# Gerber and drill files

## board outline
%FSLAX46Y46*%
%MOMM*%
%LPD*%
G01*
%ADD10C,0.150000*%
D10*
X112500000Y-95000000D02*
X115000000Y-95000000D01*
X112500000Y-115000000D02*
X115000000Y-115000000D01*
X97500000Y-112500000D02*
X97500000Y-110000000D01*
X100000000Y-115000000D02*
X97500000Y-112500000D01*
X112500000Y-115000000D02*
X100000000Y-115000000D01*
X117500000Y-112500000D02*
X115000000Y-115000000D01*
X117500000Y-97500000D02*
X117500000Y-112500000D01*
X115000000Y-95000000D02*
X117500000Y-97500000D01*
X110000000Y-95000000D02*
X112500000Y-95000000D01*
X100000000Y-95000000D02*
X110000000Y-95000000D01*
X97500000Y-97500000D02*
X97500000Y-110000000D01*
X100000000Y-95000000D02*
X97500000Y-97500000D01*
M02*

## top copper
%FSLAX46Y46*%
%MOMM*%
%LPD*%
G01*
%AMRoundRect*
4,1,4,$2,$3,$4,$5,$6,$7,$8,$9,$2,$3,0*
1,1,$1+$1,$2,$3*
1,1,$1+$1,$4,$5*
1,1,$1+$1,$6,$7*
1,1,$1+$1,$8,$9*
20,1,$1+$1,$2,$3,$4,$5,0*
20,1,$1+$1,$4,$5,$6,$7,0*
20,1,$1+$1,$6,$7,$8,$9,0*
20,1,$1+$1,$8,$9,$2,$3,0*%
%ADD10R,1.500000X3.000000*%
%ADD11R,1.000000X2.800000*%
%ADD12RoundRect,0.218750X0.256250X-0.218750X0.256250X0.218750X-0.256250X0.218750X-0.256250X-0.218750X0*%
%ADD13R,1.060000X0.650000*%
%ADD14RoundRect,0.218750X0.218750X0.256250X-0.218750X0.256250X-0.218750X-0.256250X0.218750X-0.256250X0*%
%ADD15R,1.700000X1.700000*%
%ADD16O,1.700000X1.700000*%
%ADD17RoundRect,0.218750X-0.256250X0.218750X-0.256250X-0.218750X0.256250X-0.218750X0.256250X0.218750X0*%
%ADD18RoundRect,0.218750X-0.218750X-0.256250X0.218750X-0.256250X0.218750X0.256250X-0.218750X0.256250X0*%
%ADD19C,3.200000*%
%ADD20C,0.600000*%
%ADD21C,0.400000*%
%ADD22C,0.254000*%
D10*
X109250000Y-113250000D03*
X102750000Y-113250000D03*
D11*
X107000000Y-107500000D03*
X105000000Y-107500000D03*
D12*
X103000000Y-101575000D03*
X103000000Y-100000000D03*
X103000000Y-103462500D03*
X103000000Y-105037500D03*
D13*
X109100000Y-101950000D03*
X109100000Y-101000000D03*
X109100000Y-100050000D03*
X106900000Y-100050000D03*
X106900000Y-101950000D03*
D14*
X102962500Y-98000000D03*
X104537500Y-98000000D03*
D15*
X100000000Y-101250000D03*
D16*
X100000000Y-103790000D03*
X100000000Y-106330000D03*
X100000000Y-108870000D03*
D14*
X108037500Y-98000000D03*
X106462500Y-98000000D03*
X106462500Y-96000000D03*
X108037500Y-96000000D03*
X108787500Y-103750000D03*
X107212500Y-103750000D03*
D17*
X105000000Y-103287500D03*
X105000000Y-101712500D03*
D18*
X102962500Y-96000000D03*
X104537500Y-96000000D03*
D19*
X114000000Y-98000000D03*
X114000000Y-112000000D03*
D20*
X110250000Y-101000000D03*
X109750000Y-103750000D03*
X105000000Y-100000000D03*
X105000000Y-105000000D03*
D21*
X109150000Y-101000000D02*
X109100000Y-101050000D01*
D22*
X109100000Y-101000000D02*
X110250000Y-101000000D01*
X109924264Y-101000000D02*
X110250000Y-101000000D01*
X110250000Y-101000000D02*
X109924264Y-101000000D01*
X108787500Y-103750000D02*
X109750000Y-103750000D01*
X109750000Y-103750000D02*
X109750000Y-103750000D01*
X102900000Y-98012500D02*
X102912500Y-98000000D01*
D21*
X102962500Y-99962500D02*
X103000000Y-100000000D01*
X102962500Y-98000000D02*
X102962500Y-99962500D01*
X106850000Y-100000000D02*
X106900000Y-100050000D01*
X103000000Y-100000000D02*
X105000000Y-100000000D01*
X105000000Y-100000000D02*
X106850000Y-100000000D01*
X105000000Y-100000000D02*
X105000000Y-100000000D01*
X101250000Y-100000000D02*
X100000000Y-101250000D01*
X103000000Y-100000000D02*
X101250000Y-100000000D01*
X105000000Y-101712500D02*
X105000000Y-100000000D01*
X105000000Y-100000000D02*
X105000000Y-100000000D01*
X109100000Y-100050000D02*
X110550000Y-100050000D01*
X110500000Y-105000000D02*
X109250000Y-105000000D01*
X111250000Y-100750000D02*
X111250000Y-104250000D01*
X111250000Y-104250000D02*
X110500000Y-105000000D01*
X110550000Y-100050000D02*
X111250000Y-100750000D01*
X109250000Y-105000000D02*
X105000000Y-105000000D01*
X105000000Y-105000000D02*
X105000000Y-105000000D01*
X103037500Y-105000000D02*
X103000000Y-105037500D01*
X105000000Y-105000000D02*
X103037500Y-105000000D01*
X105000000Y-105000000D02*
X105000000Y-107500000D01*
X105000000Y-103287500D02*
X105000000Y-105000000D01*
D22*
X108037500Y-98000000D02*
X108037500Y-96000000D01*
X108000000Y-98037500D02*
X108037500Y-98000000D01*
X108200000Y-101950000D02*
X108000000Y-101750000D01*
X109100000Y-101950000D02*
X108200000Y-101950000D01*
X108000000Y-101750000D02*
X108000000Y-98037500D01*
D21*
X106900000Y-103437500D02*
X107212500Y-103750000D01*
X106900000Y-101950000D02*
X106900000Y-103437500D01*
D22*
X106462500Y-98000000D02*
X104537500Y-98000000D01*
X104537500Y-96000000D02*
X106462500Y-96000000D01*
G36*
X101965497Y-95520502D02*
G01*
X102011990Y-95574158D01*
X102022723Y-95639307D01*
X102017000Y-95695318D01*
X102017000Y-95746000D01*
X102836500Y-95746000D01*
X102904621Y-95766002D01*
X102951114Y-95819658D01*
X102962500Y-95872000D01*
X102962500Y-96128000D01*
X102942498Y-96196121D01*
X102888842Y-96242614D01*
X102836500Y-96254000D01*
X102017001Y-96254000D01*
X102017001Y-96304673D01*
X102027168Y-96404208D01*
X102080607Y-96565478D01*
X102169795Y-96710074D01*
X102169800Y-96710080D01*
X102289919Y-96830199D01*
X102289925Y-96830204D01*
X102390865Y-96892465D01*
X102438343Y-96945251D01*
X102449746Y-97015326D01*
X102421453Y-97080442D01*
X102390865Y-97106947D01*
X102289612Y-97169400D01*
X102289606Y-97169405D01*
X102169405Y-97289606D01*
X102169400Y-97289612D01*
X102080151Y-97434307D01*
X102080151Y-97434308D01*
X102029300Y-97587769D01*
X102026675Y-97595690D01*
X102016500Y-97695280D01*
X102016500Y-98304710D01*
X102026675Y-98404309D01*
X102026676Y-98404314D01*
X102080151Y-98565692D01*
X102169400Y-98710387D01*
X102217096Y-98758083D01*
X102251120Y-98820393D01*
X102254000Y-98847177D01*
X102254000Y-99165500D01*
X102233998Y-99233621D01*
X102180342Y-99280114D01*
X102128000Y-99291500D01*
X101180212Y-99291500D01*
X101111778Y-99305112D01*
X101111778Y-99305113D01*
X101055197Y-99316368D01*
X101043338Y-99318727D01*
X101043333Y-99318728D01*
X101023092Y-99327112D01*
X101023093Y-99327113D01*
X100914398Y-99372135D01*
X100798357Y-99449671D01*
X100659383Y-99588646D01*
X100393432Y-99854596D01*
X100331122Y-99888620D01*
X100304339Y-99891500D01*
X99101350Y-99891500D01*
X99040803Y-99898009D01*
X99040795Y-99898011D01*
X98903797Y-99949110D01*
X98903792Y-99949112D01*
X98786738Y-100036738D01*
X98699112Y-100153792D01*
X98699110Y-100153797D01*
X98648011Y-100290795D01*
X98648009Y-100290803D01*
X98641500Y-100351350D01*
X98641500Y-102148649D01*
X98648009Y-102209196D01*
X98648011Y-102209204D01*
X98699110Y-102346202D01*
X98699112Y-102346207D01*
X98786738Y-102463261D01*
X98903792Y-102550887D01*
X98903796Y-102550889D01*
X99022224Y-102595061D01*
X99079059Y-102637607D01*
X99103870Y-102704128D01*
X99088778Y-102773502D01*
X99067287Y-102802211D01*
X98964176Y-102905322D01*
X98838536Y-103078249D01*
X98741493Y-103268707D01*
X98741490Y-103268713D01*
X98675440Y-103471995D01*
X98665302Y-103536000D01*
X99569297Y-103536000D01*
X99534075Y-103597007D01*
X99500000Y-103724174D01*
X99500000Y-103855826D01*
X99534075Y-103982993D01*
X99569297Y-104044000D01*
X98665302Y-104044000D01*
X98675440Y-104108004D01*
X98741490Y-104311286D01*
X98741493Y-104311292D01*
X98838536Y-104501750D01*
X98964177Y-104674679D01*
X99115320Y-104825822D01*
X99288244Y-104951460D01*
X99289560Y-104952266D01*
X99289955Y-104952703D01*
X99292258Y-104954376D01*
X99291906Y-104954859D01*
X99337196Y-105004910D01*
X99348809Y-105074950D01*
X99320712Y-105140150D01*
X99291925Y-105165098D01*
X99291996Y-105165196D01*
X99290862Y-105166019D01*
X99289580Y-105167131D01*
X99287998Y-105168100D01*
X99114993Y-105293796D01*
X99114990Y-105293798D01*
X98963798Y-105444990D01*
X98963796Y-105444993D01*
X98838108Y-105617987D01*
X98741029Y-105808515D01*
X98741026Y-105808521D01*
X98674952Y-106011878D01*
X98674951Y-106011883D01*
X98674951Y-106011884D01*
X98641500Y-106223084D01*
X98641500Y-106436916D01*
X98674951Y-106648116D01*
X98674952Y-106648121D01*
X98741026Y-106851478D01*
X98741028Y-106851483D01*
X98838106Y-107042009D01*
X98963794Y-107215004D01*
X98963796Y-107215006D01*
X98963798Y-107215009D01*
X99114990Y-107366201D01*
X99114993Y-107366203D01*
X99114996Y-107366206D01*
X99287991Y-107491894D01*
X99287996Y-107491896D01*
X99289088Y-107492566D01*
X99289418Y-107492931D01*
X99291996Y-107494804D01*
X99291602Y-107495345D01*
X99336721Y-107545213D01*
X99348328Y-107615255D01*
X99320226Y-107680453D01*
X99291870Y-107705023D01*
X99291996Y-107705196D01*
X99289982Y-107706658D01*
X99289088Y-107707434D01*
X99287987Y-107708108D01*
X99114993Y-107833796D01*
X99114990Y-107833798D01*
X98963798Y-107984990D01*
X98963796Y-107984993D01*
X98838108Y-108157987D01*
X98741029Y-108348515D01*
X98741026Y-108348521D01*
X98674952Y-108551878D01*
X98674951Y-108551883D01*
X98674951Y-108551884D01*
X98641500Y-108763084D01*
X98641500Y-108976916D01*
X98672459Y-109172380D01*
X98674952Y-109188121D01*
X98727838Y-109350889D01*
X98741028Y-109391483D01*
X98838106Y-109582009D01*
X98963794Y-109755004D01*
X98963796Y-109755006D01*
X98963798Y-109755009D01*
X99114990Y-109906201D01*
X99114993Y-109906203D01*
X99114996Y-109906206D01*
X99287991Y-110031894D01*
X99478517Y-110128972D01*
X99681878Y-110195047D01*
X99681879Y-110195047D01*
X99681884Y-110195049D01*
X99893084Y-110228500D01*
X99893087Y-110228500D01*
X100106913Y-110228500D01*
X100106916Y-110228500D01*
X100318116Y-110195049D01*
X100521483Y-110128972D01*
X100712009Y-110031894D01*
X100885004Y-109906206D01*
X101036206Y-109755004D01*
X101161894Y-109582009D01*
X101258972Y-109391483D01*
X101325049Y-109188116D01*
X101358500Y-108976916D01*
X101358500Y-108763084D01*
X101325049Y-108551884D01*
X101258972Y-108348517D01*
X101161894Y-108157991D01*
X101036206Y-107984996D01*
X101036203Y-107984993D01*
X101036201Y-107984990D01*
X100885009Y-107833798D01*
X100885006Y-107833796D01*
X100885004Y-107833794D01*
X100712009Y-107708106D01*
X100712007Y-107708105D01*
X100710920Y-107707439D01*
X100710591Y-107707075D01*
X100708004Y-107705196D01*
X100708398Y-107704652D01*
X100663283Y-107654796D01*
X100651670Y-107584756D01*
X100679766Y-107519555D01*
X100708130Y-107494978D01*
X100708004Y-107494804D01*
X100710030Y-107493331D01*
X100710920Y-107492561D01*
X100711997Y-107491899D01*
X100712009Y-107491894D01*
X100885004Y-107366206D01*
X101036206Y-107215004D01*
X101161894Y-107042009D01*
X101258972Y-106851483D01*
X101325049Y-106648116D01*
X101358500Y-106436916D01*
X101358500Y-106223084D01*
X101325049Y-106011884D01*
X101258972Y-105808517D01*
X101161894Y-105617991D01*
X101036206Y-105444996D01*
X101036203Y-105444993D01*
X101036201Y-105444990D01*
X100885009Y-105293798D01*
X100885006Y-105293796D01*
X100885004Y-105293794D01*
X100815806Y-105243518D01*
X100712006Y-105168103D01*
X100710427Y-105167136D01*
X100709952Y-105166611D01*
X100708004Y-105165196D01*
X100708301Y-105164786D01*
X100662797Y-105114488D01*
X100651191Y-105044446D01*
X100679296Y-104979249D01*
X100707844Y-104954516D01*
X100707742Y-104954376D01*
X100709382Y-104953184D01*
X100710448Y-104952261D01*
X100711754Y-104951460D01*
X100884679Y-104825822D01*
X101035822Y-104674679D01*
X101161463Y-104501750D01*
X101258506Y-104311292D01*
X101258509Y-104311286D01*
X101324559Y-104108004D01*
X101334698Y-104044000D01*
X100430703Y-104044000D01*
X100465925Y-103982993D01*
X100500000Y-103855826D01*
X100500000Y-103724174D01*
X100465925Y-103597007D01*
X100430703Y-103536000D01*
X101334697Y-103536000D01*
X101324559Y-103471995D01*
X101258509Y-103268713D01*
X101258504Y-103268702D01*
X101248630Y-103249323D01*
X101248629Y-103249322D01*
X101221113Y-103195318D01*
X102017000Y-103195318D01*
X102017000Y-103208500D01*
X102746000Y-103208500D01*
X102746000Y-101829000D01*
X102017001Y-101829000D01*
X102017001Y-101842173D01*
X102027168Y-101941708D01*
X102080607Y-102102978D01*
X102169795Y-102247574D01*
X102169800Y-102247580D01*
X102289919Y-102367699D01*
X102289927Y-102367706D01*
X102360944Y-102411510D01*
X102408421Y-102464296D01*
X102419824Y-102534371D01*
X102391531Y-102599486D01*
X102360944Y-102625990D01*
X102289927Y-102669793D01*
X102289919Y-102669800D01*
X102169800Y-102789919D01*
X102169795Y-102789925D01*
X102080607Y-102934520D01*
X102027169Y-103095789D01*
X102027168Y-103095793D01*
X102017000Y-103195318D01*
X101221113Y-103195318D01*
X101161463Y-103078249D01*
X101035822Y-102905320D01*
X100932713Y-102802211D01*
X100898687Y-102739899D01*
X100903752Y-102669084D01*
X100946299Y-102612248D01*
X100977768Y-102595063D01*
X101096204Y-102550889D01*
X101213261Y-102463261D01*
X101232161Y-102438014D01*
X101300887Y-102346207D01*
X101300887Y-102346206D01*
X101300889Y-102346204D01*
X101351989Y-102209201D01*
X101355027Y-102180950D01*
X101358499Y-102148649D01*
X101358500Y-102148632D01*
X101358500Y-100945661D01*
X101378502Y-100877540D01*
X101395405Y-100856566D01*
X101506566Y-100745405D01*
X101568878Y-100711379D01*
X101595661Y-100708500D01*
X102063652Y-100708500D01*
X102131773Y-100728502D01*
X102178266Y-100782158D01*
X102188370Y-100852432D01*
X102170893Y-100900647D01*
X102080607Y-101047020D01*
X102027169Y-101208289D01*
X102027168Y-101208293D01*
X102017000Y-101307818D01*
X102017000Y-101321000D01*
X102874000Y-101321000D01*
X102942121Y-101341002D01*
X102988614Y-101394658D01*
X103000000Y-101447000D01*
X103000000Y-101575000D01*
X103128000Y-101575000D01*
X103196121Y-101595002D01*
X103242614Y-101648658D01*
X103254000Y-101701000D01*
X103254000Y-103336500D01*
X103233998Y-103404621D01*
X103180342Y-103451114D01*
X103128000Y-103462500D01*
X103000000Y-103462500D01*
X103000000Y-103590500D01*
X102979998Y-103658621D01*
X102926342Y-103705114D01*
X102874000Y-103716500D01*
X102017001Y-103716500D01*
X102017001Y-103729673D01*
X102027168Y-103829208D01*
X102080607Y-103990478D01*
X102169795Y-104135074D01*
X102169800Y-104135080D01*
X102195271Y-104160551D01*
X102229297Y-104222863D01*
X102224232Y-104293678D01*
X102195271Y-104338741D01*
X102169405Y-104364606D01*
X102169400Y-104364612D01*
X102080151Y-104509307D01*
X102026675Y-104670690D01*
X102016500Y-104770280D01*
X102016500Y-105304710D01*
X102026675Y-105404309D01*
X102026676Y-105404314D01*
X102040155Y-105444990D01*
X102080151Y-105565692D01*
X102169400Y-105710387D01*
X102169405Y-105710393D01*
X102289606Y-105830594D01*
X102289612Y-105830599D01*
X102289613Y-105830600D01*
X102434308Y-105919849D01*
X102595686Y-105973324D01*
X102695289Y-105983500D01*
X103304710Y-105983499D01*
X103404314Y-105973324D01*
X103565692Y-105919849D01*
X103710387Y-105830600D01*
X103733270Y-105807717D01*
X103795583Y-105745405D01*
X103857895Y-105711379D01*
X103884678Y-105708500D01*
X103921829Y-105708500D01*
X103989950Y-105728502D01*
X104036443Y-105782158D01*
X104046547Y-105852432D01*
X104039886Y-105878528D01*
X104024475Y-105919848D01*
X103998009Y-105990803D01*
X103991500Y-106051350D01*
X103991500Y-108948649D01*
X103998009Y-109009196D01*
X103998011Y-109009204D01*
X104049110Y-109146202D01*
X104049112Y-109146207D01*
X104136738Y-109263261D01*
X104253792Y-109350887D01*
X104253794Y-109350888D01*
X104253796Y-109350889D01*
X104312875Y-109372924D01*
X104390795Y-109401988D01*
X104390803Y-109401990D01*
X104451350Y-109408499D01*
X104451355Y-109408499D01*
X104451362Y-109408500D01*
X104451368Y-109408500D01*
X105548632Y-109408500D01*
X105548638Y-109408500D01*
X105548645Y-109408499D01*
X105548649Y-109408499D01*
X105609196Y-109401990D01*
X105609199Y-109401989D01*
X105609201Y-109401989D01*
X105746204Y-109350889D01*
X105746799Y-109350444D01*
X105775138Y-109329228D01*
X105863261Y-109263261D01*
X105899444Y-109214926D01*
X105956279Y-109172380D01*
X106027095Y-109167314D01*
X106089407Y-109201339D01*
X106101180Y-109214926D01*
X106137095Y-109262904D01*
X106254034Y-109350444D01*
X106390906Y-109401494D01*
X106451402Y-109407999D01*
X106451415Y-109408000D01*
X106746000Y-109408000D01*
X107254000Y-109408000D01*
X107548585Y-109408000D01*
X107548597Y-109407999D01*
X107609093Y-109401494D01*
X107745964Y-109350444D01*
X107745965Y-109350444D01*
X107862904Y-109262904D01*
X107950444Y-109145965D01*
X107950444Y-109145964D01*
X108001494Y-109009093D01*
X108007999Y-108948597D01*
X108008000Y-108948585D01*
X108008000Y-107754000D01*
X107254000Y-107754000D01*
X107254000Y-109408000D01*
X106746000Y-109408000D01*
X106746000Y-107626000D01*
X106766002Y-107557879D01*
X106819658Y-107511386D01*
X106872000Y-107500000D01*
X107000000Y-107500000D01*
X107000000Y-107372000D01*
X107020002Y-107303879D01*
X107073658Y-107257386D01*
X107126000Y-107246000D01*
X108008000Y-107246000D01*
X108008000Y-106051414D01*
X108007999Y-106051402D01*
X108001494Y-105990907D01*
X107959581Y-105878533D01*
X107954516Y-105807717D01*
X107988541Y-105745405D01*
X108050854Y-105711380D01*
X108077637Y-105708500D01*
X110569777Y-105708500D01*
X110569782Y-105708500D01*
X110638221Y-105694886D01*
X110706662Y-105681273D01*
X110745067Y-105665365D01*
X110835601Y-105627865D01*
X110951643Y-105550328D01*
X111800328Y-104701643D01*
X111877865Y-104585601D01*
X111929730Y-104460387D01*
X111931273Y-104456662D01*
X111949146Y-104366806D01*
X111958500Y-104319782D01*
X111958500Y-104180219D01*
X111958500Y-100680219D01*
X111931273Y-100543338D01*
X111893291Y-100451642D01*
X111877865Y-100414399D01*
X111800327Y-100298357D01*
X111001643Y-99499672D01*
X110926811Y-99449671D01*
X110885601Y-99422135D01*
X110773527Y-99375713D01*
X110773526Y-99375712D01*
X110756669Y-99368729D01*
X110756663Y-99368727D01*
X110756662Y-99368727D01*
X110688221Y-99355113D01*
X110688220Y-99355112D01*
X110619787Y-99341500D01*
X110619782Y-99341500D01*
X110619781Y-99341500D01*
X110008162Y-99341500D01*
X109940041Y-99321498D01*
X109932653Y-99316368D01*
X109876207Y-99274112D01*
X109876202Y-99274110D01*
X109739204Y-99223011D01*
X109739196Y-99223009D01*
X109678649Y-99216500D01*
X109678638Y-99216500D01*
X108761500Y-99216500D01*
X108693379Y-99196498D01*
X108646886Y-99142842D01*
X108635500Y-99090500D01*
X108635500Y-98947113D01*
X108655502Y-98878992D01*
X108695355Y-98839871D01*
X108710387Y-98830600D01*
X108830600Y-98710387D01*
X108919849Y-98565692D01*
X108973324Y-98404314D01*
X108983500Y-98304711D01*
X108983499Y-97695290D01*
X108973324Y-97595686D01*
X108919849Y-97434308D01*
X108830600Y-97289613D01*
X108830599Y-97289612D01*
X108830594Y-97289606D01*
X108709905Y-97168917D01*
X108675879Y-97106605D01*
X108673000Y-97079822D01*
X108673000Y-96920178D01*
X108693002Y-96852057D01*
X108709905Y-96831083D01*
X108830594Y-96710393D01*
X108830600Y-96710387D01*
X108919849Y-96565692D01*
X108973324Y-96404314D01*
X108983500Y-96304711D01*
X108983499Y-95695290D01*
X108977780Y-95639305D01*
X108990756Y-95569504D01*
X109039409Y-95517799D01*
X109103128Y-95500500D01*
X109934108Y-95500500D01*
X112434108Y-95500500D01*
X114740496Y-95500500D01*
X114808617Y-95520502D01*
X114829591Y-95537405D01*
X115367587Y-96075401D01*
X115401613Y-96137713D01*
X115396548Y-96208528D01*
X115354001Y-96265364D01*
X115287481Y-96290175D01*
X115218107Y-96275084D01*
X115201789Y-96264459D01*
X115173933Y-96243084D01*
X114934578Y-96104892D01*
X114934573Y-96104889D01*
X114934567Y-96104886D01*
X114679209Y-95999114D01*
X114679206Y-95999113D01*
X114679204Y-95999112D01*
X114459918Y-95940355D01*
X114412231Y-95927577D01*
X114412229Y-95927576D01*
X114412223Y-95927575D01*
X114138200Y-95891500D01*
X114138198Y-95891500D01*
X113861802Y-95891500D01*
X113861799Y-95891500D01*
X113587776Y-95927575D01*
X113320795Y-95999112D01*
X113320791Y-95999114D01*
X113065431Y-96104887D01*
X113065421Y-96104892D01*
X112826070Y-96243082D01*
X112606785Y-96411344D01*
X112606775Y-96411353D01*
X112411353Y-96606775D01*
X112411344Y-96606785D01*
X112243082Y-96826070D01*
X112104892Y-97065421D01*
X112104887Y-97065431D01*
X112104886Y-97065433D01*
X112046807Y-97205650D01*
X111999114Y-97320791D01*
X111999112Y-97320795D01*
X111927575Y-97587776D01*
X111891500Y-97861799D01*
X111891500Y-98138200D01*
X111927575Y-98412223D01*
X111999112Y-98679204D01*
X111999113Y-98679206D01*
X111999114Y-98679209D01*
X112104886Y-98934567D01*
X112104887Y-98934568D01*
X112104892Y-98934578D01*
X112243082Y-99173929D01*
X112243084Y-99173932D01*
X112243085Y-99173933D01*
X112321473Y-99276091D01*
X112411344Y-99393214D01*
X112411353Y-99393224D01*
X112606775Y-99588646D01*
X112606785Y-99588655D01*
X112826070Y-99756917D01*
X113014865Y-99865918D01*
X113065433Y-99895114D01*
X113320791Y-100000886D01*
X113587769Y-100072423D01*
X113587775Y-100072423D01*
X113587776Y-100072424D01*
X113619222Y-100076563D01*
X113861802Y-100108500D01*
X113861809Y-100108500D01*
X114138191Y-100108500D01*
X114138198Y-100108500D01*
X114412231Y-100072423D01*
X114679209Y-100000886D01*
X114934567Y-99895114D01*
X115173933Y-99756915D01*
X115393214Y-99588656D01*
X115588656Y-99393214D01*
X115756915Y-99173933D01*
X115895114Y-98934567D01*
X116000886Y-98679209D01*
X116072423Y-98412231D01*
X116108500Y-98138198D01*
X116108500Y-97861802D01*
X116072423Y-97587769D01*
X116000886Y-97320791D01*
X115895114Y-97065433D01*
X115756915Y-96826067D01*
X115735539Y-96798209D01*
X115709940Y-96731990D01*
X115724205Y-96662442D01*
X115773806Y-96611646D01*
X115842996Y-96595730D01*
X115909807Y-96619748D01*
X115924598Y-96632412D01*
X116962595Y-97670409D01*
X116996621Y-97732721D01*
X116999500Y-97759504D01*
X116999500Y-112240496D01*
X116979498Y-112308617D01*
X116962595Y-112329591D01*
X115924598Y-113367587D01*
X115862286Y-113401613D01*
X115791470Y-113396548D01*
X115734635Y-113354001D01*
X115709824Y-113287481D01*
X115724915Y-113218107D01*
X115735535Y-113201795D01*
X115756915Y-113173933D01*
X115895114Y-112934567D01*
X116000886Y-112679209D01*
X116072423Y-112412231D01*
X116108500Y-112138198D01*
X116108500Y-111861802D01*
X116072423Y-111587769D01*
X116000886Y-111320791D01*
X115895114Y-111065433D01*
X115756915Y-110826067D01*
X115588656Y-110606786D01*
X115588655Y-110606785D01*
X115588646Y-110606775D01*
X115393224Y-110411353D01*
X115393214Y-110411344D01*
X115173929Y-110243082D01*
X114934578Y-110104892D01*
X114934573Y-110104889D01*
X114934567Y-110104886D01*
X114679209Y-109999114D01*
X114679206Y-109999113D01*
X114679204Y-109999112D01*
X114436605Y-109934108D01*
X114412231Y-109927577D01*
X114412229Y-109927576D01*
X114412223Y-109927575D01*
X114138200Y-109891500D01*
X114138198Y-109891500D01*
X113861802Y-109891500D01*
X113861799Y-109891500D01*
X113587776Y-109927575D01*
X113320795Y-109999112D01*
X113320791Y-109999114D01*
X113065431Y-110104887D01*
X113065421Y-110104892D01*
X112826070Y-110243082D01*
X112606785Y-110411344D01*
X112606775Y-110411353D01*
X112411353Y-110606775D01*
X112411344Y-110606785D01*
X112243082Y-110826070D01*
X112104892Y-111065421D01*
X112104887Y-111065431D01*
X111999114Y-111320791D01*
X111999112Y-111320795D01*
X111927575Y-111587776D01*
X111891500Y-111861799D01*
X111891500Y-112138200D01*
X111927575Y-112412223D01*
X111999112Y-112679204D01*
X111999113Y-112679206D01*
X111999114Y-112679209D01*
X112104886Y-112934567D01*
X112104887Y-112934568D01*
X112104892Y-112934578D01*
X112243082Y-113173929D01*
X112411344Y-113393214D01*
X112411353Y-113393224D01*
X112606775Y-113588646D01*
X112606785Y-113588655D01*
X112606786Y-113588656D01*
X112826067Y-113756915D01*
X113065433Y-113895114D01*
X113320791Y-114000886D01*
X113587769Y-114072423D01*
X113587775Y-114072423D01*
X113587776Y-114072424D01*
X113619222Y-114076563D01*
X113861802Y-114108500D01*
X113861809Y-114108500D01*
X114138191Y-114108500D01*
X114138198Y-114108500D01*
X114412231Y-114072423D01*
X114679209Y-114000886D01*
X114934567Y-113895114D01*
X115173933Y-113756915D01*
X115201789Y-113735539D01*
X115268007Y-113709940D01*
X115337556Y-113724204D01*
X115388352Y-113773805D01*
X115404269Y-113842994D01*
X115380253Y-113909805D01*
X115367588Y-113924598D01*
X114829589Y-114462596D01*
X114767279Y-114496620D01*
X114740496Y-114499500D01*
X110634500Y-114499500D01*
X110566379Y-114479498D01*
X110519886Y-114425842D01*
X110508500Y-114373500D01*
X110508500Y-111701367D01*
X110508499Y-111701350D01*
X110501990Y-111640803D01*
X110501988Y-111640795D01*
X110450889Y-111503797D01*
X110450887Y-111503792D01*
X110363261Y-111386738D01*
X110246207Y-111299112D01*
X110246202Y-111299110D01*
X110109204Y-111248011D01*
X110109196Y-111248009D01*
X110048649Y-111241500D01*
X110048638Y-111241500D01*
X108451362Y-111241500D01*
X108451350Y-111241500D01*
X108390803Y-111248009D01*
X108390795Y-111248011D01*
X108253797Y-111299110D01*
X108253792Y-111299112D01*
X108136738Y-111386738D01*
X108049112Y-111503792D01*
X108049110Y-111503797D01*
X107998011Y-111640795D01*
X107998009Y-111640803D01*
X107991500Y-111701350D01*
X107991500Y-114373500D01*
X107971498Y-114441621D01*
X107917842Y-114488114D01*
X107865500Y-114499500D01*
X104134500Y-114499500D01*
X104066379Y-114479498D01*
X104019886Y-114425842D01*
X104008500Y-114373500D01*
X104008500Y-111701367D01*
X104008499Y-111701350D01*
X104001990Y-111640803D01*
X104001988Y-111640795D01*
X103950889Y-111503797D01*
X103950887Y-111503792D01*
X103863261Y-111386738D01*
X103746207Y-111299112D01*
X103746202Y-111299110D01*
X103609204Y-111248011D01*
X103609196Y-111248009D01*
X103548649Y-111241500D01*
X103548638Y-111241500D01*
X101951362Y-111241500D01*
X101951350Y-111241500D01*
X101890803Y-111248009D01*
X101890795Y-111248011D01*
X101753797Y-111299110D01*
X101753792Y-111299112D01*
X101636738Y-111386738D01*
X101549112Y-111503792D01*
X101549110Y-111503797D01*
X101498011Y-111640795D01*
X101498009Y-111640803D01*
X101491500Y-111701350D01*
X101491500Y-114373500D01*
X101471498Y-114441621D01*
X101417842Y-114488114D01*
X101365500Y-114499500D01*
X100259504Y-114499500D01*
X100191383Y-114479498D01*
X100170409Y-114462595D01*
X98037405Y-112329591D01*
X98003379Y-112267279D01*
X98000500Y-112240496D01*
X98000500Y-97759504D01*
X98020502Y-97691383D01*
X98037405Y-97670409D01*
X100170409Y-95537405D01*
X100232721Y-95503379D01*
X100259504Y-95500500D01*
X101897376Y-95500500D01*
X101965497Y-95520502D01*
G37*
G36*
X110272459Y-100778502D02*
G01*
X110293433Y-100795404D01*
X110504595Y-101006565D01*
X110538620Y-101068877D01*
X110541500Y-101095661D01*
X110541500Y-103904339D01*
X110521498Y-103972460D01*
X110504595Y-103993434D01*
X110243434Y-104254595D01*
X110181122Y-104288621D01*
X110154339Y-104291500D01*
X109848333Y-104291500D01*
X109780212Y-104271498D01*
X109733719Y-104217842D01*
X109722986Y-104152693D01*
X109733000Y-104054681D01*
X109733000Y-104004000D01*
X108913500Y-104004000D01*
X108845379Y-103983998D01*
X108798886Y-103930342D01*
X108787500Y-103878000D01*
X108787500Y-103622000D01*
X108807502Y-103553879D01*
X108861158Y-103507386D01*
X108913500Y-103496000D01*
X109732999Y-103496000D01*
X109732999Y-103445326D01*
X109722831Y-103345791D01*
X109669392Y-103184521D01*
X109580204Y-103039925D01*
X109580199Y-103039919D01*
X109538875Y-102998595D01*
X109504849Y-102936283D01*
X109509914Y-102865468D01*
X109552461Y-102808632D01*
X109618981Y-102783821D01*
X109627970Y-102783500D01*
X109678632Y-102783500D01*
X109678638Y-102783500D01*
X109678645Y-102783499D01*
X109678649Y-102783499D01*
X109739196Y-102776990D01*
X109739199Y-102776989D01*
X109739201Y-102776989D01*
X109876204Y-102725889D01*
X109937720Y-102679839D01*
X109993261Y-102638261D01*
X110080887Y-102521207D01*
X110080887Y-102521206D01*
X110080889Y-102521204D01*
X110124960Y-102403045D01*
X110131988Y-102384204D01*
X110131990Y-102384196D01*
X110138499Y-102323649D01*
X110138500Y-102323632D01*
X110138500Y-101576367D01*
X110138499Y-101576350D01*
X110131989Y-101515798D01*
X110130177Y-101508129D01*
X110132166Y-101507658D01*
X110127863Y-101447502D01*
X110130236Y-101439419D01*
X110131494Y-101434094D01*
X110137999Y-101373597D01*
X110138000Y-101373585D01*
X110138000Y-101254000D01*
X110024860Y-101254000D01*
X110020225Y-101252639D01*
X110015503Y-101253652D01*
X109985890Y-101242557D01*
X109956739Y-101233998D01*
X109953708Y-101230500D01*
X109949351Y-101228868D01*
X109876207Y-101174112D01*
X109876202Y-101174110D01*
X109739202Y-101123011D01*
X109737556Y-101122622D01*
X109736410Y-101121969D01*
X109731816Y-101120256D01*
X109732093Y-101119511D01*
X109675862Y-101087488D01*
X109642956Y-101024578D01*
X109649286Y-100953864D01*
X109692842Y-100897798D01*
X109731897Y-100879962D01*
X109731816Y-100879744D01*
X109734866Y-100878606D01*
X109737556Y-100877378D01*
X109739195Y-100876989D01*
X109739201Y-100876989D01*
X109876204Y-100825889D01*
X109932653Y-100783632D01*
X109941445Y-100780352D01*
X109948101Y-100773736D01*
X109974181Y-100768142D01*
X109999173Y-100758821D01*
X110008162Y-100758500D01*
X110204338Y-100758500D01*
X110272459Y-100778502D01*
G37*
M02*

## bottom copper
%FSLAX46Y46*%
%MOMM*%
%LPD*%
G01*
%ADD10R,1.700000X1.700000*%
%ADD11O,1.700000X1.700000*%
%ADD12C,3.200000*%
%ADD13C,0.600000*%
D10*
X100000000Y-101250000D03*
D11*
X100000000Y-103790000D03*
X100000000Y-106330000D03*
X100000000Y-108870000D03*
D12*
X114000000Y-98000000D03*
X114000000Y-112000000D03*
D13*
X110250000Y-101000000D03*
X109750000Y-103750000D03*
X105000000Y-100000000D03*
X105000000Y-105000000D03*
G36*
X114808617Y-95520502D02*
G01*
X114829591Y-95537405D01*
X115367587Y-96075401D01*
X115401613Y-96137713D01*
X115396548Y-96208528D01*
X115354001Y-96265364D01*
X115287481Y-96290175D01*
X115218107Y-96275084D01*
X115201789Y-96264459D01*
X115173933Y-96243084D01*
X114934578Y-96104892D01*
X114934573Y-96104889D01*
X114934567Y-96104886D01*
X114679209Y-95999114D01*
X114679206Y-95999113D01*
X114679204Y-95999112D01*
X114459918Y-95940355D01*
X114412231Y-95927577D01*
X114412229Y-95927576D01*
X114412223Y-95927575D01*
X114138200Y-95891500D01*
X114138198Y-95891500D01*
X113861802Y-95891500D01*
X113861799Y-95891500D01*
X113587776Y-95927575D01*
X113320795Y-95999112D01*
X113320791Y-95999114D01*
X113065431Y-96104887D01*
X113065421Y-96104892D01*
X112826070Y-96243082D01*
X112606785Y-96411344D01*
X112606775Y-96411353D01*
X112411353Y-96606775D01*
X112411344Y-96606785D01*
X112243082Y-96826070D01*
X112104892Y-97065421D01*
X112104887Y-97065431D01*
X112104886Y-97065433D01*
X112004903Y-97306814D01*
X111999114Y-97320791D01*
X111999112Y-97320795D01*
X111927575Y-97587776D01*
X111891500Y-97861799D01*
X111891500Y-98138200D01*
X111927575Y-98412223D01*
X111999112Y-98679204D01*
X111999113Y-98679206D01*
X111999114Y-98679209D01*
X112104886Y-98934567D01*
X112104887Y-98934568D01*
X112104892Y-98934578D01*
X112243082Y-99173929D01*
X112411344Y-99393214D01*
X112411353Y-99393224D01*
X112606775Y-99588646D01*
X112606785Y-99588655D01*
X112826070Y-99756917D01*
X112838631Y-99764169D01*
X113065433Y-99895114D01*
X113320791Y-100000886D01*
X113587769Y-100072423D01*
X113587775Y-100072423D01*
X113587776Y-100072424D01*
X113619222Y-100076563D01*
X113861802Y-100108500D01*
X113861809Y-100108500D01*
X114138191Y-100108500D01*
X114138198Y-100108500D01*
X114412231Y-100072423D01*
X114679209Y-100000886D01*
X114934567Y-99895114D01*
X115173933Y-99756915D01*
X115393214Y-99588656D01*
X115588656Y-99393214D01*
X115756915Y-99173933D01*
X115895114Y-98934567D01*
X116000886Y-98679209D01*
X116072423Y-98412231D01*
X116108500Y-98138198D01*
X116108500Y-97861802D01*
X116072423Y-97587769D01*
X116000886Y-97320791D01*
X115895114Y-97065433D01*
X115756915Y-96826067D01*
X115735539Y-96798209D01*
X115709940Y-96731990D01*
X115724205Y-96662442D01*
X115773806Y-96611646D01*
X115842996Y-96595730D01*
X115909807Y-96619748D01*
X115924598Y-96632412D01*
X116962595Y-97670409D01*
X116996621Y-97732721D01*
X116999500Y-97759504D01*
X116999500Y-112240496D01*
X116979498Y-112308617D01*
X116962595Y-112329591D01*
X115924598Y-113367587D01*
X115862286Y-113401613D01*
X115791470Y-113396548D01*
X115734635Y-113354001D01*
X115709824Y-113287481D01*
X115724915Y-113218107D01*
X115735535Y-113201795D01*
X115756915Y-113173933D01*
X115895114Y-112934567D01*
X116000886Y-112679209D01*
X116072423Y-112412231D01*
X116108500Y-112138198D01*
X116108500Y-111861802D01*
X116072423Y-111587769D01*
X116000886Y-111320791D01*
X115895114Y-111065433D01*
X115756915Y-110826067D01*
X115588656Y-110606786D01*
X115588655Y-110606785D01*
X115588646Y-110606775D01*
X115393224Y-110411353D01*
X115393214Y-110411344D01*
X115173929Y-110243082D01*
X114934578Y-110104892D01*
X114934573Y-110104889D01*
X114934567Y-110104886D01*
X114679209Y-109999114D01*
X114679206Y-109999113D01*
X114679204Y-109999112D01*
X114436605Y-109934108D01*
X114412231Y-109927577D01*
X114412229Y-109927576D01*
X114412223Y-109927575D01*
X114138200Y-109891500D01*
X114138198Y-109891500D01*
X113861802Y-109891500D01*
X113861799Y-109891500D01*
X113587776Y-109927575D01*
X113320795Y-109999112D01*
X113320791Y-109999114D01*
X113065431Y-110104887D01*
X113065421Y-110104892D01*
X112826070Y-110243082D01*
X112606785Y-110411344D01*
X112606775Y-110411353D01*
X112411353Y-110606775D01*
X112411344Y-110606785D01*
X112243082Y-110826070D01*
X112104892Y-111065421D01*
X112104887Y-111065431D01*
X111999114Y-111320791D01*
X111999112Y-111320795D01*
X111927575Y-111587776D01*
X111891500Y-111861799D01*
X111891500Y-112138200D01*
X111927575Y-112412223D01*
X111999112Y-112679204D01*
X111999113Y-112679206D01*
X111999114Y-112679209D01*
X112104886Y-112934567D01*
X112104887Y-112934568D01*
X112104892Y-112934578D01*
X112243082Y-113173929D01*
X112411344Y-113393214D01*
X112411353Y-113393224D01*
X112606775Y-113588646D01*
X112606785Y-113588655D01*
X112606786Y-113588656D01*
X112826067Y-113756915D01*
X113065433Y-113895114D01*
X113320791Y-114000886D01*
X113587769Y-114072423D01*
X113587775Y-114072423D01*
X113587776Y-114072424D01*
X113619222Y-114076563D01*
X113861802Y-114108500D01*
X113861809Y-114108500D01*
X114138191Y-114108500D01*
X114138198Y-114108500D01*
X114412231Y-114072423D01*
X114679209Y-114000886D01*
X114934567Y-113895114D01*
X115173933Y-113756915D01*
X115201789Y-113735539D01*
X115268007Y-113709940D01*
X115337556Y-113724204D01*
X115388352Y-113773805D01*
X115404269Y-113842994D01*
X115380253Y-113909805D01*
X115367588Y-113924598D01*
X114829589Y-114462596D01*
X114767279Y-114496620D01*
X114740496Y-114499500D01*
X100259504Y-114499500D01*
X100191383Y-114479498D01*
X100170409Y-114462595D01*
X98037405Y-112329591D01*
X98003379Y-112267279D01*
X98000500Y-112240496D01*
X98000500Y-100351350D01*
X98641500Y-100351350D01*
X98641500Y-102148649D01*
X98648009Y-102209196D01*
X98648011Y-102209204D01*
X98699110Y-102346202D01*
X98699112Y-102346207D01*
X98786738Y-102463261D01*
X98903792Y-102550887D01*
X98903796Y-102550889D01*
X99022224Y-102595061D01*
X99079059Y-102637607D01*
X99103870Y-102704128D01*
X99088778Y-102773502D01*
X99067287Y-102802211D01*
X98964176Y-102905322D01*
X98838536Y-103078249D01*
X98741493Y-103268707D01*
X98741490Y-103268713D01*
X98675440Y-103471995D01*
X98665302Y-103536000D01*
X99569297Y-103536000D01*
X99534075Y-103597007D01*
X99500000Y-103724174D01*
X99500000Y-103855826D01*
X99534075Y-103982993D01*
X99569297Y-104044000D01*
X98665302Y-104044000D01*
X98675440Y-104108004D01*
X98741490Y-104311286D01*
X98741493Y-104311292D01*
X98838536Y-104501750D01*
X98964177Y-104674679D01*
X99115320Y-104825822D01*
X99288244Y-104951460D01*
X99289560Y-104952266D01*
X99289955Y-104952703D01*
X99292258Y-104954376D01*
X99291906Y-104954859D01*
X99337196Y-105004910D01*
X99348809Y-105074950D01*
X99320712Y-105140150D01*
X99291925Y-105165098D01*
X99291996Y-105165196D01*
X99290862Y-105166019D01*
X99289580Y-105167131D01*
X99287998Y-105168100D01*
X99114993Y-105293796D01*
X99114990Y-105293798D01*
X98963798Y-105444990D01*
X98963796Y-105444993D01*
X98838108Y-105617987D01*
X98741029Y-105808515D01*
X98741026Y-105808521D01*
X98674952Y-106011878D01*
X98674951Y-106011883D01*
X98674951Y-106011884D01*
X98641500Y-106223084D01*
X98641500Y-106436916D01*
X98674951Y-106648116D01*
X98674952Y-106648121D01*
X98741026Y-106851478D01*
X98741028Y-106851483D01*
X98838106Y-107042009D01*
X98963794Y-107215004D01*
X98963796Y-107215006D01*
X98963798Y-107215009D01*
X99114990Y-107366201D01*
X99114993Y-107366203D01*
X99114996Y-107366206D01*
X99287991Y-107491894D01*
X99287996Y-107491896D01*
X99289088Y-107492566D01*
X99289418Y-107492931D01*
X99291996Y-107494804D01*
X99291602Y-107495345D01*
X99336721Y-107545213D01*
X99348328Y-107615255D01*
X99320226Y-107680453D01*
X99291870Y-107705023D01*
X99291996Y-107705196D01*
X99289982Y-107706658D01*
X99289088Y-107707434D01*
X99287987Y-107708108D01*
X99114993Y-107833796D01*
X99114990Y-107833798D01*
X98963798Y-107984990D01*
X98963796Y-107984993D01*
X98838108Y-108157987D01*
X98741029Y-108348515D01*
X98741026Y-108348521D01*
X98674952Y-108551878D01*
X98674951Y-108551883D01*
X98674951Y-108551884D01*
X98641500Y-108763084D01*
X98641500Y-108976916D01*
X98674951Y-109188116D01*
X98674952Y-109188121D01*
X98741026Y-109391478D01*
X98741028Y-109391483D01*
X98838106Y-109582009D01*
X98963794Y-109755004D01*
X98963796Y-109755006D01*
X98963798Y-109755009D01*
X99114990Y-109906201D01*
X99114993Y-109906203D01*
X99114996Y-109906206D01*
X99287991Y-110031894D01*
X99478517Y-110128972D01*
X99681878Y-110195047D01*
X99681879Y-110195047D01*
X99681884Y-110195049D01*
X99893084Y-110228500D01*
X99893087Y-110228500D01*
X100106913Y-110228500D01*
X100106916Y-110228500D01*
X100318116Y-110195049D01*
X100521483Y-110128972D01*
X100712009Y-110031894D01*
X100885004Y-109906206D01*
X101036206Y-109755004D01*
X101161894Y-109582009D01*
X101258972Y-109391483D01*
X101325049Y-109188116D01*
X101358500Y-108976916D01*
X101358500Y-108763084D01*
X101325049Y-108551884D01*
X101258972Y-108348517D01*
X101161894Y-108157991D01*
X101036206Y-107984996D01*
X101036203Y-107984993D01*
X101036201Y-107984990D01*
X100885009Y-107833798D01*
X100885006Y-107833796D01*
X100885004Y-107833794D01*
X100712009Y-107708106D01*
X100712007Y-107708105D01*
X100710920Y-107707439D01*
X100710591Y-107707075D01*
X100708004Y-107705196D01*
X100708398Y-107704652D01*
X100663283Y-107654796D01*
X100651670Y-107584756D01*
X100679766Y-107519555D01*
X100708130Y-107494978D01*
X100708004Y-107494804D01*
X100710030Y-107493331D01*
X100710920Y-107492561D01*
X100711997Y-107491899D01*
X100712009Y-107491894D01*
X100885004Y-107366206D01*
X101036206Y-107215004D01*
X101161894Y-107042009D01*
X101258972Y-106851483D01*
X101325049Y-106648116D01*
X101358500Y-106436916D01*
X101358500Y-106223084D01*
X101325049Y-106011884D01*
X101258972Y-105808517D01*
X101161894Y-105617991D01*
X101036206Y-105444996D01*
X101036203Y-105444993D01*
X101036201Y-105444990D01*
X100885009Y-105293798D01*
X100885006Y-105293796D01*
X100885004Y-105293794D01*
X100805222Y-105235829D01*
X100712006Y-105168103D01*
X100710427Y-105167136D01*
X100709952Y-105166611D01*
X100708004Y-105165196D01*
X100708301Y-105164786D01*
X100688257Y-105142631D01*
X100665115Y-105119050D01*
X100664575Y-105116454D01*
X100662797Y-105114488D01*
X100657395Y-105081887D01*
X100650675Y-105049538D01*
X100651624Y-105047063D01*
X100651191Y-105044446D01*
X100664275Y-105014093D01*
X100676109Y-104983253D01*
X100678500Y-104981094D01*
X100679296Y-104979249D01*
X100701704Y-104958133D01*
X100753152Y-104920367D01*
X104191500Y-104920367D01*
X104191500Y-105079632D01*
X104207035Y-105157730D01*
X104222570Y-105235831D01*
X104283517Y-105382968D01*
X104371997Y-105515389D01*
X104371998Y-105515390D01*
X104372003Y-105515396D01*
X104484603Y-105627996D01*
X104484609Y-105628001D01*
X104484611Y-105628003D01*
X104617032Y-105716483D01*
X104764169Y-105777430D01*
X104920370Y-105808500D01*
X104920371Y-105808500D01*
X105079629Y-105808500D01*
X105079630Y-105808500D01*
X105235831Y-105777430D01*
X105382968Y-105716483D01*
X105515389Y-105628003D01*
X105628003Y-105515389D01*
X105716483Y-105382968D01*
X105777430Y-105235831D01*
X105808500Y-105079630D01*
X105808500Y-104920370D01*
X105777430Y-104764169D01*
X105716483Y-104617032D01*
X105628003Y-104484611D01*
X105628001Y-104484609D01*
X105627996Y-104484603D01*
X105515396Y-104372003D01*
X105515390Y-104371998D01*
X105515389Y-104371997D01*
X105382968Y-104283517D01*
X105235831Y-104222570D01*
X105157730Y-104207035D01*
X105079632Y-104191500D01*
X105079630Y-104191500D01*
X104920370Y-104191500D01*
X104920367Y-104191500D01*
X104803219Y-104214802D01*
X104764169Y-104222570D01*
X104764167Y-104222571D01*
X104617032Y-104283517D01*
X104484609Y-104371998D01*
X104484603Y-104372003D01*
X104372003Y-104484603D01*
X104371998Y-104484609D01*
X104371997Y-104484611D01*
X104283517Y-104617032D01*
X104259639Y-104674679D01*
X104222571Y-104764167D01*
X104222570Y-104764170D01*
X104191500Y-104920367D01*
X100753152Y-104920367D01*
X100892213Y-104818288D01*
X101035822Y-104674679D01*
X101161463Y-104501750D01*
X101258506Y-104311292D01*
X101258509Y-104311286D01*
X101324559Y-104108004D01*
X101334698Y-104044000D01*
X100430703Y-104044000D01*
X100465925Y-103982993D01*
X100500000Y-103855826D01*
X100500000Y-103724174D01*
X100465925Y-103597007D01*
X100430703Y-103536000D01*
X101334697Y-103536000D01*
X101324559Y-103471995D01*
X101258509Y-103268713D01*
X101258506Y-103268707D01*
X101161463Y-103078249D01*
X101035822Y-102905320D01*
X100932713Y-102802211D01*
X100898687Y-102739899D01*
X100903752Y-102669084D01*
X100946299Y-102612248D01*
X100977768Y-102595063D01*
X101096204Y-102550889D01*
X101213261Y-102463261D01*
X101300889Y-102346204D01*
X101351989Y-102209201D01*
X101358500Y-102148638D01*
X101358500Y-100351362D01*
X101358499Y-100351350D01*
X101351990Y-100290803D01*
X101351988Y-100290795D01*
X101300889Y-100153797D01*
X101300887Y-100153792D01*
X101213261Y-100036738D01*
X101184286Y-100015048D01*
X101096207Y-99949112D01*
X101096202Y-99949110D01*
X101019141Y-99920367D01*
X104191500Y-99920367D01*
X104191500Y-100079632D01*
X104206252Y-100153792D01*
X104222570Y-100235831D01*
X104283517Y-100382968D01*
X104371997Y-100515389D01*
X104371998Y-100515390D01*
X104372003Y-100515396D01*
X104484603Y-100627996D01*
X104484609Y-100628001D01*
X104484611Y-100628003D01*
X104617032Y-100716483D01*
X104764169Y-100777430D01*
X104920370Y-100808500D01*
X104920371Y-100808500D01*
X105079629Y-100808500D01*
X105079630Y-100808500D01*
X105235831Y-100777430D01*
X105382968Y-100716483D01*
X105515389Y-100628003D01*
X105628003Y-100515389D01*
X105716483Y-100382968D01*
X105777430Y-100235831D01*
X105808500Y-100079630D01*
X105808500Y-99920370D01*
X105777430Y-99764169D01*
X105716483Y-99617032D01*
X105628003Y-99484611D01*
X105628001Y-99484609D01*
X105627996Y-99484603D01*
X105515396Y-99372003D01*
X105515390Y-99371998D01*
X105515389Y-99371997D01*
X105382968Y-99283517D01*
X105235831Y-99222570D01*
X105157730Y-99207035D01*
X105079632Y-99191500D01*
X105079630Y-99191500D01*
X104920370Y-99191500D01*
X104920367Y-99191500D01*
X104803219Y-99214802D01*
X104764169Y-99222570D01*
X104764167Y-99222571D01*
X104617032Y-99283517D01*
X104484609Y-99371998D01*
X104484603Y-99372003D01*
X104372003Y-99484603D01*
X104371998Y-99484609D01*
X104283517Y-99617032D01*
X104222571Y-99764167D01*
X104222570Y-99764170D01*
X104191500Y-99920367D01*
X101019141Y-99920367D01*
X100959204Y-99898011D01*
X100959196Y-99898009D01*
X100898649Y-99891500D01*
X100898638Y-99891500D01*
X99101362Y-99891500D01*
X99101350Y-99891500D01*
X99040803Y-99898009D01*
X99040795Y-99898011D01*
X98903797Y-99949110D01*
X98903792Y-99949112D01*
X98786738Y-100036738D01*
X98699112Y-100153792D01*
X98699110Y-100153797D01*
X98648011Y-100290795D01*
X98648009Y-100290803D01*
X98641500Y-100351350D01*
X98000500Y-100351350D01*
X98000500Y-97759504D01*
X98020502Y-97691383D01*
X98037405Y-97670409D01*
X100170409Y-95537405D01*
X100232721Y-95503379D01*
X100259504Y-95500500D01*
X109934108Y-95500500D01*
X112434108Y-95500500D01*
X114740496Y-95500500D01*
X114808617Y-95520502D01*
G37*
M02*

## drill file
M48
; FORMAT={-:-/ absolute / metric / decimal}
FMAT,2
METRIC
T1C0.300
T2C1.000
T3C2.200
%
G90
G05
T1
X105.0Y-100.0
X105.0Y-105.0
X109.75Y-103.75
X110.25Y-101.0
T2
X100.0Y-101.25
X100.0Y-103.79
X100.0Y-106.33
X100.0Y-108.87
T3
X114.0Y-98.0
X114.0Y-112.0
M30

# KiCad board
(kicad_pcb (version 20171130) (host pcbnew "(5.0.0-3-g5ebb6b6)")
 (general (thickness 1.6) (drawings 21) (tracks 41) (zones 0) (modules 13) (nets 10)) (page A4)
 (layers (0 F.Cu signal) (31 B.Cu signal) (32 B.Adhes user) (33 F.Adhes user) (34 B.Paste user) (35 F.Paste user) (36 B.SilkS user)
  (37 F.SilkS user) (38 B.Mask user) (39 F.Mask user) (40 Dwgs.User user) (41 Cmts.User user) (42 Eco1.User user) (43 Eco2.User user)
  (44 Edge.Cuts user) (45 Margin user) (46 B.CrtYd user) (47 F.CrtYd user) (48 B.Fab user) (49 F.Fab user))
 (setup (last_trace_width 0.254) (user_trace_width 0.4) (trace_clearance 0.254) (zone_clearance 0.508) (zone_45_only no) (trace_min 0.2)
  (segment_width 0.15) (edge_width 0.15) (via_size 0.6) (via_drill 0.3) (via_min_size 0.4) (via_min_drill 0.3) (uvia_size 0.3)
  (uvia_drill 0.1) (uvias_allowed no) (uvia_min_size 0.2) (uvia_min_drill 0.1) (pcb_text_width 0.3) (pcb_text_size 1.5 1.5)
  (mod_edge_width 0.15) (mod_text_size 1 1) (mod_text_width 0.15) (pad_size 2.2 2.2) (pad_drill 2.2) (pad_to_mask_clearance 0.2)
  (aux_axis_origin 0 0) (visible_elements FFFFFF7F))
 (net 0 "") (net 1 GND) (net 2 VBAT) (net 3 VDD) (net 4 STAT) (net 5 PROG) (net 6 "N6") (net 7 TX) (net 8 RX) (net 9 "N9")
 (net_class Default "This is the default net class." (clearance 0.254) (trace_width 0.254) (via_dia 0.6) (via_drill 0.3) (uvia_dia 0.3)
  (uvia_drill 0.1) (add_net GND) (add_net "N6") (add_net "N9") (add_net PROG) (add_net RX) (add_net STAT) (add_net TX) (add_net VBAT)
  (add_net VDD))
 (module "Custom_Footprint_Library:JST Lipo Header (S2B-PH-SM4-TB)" (layer F.Cu) (at 106 112)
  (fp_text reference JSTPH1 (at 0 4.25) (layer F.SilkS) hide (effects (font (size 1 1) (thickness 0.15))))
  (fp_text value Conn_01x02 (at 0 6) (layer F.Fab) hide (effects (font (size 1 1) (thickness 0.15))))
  (pad "" connect rect (at 3.25 1.25) (size 1.5 3) (layers F.Cu F.Mask))
  (pad "" connect rect (at -3.25 1.25) (size 1.5 3) (layers F.Cu F.Mask))
  (pad 2 smd rect (at 1 -4.5) (size 1 2.8) (layers F.Cu F.Paste F.Mask) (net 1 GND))
  (pad 1 smd rect (at -1 -4.5) (size 1 2.8) (layers F.Cu F.Paste F.Mask) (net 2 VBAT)))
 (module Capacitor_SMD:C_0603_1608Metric (layer F.Cu) (at 103 100.7875 90)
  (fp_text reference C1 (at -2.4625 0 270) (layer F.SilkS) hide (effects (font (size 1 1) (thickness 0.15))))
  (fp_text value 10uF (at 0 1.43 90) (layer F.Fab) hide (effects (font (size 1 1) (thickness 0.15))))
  (pad 1 smd roundrect (at -0.7875 0 90) (size 0.875 0.95) (layers F.Cu F.Paste F.Mask) (roundrect_rratio 0.25) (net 1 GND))
  (pad 2 smd roundrect (at 0.7875 0 90) (size 0.875 0.95) (layers F.Cu F.Paste F.Mask) (roundrect_rratio 0.25) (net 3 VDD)))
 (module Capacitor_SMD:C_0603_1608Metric (layer F.Cu) (at 103 104.25 90)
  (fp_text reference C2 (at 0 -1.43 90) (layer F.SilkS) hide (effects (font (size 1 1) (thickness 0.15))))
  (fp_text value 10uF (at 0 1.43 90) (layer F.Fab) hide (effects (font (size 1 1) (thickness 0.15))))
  (pad 2 smd roundrect (at 0.7875 0 90) (size 0.875 0.95) (layers F.Cu F.Paste F.Mask) (roundrect_rratio 0.25) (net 1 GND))
  (pad 1 smd roundrect (at -0.7875 0 90) (size 0.875 0.95) (layers F.Cu F.Paste F.Mask) (roundrect_rratio 0.25) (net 2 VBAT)))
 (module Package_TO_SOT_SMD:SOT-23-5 (layer F.Cu) (at 108 101 180)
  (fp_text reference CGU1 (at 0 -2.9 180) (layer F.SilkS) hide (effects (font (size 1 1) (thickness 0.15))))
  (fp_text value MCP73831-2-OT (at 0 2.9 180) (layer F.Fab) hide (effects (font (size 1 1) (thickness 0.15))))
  (pad 1 smd rect (at -1.1 -0.95 180) (size 1.06 0.65) (layers F.Cu F.Paste F.Mask) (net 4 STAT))
  (pad 2 smd rect (at -1.1 0 180) (size 1.06 0.65) (layers F.Cu F.Paste F.Mask) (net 1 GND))
  (pad 3 smd rect (at -1.1 0.95 180) (size 1.06 0.65) (layers F.Cu F.Paste F.Mask) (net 2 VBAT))
  (pad 4 smd rect (at 1.1 0.95 180) (size 1.06 0.65) (layers F.Cu F.Paste F.Mask) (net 3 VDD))
  (pad 5 smd rect (at 1.1 -0.95 180) (size 1.06 0.65) (layers F.Cu F.Paste F.Mask) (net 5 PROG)))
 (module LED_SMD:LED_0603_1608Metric (layer F.Cu) (at 103.75 98 180)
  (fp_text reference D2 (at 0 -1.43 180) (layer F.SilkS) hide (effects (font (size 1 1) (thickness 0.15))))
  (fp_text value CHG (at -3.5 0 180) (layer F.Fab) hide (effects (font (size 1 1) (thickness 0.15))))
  (pad 2 smd roundrect (at 0.7875 0 180) (size 0.875 0.95) (layers F.Cu F.Paste F.Mask) (roundrect_rratio 0.25) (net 3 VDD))
  (pad 1 smd roundrect (at -0.7875 0 180) (size 0.875 0.95) (layers F.Cu F.Paste F.Mask) (roundrect_rratio 0.25) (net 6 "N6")))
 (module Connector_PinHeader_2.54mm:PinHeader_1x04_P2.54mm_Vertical (layer F.Cu) (at 100 101.25)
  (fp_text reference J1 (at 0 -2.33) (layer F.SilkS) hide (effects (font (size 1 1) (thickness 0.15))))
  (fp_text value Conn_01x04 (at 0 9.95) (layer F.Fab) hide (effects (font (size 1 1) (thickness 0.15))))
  (pad 1 thru_hole rect (at 0 0) (size 1.7 1.7) (drill 1) (layers *.Cu *.Mask) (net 3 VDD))
  (pad 2 thru_hole oval (at 0 2.54) (size 1.7 1.7) (drill 1) (layers *.Cu *.Mask) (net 1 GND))
  (pad 3 thru_hole oval (at 0 5.08) (size 1.7 1.7) (drill 1) (layers *.Cu *.Mask) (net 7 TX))
  (pad 4 thru_hole oval (at 0 7.62) (size 1.7 1.7) (drill 1) (layers *.Cu *.Mask) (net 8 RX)))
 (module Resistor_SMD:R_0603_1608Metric (layer F.Cu) (at 107.25 98 180)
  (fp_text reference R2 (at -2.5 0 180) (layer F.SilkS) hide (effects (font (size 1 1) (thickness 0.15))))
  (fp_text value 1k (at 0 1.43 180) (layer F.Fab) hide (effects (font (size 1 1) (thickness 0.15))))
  (pad 1 smd roundrect (at -0.7875 0 180) (size 0.875 0.95) (layers F.Cu F.Paste F.Mask) (roundrect_rratio 0.25) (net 4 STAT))
  (pad 2 smd roundrect (at 0.7875 0 180) (size 0.875 0.95) (layers F.Cu F.Paste F.Mask) (roundrect_rratio 0.25) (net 6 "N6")))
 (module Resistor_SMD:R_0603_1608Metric (layer F.Cu) (at 107.25 96 180)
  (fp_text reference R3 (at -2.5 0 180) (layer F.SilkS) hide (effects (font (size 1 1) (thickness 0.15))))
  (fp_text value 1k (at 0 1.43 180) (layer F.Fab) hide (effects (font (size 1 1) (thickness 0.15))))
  (pad 2 smd roundrect (at 0.7875 0 180) (size 0.875 0.95) (layers F.Cu F.Paste F.Mask) (roundrect_rratio 0.25) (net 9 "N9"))
  (pad 1 smd roundrect (at -0.7875 0 180) (size 0.875 0.95) (layers F.Cu F.Paste F.Mask) (roundrect_rratio 0.25) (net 4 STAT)))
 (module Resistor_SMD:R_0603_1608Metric (layer F.Cu) (at 108 103.75 180)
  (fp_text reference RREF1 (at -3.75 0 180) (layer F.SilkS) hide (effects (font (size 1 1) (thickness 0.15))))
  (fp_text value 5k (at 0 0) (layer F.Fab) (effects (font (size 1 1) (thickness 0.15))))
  (pad 1 smd roundrect (at -0.7875 0 180) (size 0.875 0.95) (layers F.Cu F.Paste F.Mask) (roundrect_rratio 0.25) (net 1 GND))
  (pad 2 smd roundrect (at 0.7875 0 180) (size 0.875 0.95) (layers F.Cu F.Paste F.Mask) (roundrect_rratio 0.25) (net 5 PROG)))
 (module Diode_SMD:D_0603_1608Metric (layer F.Cu) (at 105 102.5 270)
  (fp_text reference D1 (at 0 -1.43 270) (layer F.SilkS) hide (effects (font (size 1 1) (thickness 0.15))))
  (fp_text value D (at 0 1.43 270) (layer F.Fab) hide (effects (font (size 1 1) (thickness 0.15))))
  (pad 2 smd roundrect (at 0.7875 0 270) (size 0.875 0.95) (layers F.Cu F.Paste F.Mask) (roundrect_rratio 0.25) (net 2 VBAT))
  (pad 1 smd roundrect (at -0.7875 0 270) (size 0.875 0.95) (layers F.Cu F.Paste F.Mask) (roundrect_rratio 0.25) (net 3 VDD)))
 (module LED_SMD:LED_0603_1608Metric (layer F.Cu) (at 103.75 96)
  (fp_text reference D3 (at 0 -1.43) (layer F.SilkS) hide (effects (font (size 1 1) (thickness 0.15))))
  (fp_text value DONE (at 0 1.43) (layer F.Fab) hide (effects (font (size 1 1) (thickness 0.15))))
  (pad 1 smd roundrect (at -0.7875 0) (size 0.875 0.95) (layers F.Cu F.Paste F.Mask) (roundrect_rratio 0.25) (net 1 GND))
  (pad 2 smd roundrect (at 0.7875 0) (size 0.875 0.95) (layers F.Cu F.Paste F.Mask) (roundrect_rratio 0.25) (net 9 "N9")))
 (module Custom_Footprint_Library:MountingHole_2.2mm (layer F.Cu) (at 114 98)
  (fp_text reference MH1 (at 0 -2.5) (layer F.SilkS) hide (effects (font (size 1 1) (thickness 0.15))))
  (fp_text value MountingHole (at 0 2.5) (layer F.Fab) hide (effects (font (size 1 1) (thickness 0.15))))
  (pad "" thru_hole circle (at 0 0) (size 3.2 3.2) (drill 2.2) (layers *.Cu *.Mask)))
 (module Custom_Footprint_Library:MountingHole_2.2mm (layer F.Cu) (at 114 112)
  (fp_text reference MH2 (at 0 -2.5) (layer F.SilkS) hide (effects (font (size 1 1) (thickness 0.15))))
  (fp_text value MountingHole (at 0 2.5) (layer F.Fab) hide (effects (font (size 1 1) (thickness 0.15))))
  (pad "" thru_hole circle (at 0 0) (size 3.2 3.2) (drill 2.2) (layers *.Cu *.Mask)))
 (gr_line (start 112.5 95) (end 115 95) (layer Edge.Cuts) (width 0.15))
 (gr_line (start 112.5 115) (end 115 115) (layer Edge.Cuts) (width 0.15))
 (gr_line (start 97.5 112.5) (end 97.5 110) (layer Edge.Cuts) (width 0.15))
 (gr_line (start 100 115) (end 97.5 112.5) (layer Edge.Cuts) (width 0.15))
 (gr_line (start 112.5 115) (end 100 115) (layer Edge.Cuts) (width 0.15))
 (gr_line (start 117.5 112.5) (end 115 115) (layer Edge.Cuts) (width 0.15))
 (gr_line (start 117.5 97.5) (end 117.5 112.5) (layer Edge.Cuts) (width 0.15))
 (gr_line (start 115 95) (end 117.5 97.5) (layer Edge.Cuts) (width 0.15))
 (gr_line (start 110 95) (end 112.5 95) (layer Edge.Cuts) (width 0.15))
 (gr_line (start 100 95) (end 110 95) (layer Edge.Cuts) (width 0.15))
 (gr_line (start 97.5 97.5) (end 97.5 110) (layer Edge.Cuts) (width 0.15))
 (gr_line (start 100 95) (end 97.5 97.5) (layer Edge.Cuts) (width 0.15))
 (segment (start 109.15 101) (end 109.1 101.05) (width 0.4) (layer F.Cu) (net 1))
 (segment (start 109.1 101) (end 110.25 101) (width 0.254) (layer F.Cu) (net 1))
 (segment (start 109.924264 101) (end 110.25 101) (width 0.254) (layer F.Cu) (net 1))
 (segment (start 110.25 101) (end 109.924264 101) (width 0.254) (layer F.Cu) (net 1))
 (via (at 110.25 101) (size 0.6) (drill 0.3) (layers F.Cu B.Cu) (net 1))
 (segment (start 108.7875 103.75) (end 109.75 103.75) (width 0.254) (layer F.Cu) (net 1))
 (segment (start 109.75 103.75) (end 109.75 103.75) (width 0.254) (layer F.Cu) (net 1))
 (via (at 109.75 103.75) (size 0.6) (drill 0.3) (layers F.Cu B.Cu) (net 1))
 (segment (start 102.9 98.0125) (end 102.9125 98) (width 0.254) (layer F.Cu) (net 3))
 (segment (start 102.9625 99.9625) (end 103 100) (width 0.4) (layer F.Cu) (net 3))
 (segment (start 102.9625 98) (end 102.9625 99.9625) (width 0.4) (layer F.Cu) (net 3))
 (segment (start 106.85 100) (end 106.9 100.05) (width 0.4) (layer F.Cu) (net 3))
 (segment (start 103 100) (end 105 100) (width 0.4) (layer F.Cu) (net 3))
 (segment (start 105 100) (end 106.85 100) (width 0.4) (layer F.Cu) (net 3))
 (segment (start 105 100) (end 105 100) (width 0.4) (layer F.Cu) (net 3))
 (segment (start 101.25 100) (end 100 101.25) (width 0.4) (layer F.Cu) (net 3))
 (segment (start 103 100) (end 101.25 100) (width 0.4) (layer F.Cu) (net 3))
 (segment (start 105 101.7125) (end 105 100) (width 0.4) (layer F.Cu) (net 3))
 (segment (start 105 100) (end 105 100) (width 0.4) (layer F.Cu) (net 3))
 (via (at 105 100) (size 0.6) (drill 0.3) (layers F.Cu B.Cu) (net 3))
 (segment (start 109.1 100.05) (end 110.55 100.05) (width 0.4) (layer F.Cu) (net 2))
 (segment (start 110.5 105) (end 109.25 105) (width 0.4) (layer F.Cu) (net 2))
 (segment (start 111.25 100.75) (end 111.25 104.25) (width 0.4) (layer F.Cu) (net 2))
 (segment (start 111.25 104.25) (end 110.5 105) (width 0.4) (layer F.Cu) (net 2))
 (segment (start 110.55 100.05) (end 111.25 100.75) (width 0.4) (layer F.Cu) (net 2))
 (segment (start 109.25 105) (end 105 105) (width 0.4) (layer F.Cu) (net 2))
 (segment (start 105 105) (end 105 105) (width 0.4) (layer F.Cu) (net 2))
 (via (at 105 105) (size 0.6) (drill 0.3) (layers F.Cu B.Cu) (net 2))
 (segment (start 103.0375 105) (end 103 105.0375) (width 0.4) (layer F.Cu) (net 2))
 (segment (start 105 105) (end 103.0375 105) (width 0.4) (layer F.Cu) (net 2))
 (segment (start 105 105) (end 105 107.5) (width 0.4) (layer F.Cu) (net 2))
 (segment (start 105 103.2875) (end 105 105) (width 0.4) (layer F.Cu) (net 2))
 (segment (start 108.0375 98) (end 108.0375 96) (width 0.254) (layer F.Cu) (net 4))
 (segment (start 108 98.0375) (end 108.0375 98) (width 0.254) (layer F.Cu) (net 4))
 (segment (start 108.2 101.95) (end 108 101.75) (width 0.254) (layer F.Cu) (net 4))
 (segment (start 109.1 101.95) (end 108.2 101.95) (width 0.254) (layer F.Cu) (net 4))
 (segment (start 108 101.75) (end 108 98.0375) (width 0.254) (layer F.Cu) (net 4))
 (segment (start 106.9 103.4375) (end 107.2125 103.75) (width 0.4) (layer F.Cu) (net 5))
 (segment (start 106.9 101.95) (end 106.9 103.4375) (width 0.4) (layer F.Cu) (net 5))
 (segment (start 106.4625 98) (end 104.5375 98) (width 0.254) (layer F.Cu) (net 6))
 (segment (start 104.5375 96) (end 106.4625 96) (width 0.254) (layer F.Cu) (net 9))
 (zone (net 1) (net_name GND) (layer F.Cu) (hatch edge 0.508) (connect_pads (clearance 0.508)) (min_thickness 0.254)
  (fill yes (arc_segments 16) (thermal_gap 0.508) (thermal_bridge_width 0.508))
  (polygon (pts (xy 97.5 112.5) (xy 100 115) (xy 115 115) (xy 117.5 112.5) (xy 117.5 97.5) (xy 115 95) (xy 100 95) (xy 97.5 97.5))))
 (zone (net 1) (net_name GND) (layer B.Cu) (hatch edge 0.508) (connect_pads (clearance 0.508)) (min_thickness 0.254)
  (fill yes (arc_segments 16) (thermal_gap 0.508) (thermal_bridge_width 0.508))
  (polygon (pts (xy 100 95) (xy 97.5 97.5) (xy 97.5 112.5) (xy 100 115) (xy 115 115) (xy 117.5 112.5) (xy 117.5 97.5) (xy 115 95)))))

